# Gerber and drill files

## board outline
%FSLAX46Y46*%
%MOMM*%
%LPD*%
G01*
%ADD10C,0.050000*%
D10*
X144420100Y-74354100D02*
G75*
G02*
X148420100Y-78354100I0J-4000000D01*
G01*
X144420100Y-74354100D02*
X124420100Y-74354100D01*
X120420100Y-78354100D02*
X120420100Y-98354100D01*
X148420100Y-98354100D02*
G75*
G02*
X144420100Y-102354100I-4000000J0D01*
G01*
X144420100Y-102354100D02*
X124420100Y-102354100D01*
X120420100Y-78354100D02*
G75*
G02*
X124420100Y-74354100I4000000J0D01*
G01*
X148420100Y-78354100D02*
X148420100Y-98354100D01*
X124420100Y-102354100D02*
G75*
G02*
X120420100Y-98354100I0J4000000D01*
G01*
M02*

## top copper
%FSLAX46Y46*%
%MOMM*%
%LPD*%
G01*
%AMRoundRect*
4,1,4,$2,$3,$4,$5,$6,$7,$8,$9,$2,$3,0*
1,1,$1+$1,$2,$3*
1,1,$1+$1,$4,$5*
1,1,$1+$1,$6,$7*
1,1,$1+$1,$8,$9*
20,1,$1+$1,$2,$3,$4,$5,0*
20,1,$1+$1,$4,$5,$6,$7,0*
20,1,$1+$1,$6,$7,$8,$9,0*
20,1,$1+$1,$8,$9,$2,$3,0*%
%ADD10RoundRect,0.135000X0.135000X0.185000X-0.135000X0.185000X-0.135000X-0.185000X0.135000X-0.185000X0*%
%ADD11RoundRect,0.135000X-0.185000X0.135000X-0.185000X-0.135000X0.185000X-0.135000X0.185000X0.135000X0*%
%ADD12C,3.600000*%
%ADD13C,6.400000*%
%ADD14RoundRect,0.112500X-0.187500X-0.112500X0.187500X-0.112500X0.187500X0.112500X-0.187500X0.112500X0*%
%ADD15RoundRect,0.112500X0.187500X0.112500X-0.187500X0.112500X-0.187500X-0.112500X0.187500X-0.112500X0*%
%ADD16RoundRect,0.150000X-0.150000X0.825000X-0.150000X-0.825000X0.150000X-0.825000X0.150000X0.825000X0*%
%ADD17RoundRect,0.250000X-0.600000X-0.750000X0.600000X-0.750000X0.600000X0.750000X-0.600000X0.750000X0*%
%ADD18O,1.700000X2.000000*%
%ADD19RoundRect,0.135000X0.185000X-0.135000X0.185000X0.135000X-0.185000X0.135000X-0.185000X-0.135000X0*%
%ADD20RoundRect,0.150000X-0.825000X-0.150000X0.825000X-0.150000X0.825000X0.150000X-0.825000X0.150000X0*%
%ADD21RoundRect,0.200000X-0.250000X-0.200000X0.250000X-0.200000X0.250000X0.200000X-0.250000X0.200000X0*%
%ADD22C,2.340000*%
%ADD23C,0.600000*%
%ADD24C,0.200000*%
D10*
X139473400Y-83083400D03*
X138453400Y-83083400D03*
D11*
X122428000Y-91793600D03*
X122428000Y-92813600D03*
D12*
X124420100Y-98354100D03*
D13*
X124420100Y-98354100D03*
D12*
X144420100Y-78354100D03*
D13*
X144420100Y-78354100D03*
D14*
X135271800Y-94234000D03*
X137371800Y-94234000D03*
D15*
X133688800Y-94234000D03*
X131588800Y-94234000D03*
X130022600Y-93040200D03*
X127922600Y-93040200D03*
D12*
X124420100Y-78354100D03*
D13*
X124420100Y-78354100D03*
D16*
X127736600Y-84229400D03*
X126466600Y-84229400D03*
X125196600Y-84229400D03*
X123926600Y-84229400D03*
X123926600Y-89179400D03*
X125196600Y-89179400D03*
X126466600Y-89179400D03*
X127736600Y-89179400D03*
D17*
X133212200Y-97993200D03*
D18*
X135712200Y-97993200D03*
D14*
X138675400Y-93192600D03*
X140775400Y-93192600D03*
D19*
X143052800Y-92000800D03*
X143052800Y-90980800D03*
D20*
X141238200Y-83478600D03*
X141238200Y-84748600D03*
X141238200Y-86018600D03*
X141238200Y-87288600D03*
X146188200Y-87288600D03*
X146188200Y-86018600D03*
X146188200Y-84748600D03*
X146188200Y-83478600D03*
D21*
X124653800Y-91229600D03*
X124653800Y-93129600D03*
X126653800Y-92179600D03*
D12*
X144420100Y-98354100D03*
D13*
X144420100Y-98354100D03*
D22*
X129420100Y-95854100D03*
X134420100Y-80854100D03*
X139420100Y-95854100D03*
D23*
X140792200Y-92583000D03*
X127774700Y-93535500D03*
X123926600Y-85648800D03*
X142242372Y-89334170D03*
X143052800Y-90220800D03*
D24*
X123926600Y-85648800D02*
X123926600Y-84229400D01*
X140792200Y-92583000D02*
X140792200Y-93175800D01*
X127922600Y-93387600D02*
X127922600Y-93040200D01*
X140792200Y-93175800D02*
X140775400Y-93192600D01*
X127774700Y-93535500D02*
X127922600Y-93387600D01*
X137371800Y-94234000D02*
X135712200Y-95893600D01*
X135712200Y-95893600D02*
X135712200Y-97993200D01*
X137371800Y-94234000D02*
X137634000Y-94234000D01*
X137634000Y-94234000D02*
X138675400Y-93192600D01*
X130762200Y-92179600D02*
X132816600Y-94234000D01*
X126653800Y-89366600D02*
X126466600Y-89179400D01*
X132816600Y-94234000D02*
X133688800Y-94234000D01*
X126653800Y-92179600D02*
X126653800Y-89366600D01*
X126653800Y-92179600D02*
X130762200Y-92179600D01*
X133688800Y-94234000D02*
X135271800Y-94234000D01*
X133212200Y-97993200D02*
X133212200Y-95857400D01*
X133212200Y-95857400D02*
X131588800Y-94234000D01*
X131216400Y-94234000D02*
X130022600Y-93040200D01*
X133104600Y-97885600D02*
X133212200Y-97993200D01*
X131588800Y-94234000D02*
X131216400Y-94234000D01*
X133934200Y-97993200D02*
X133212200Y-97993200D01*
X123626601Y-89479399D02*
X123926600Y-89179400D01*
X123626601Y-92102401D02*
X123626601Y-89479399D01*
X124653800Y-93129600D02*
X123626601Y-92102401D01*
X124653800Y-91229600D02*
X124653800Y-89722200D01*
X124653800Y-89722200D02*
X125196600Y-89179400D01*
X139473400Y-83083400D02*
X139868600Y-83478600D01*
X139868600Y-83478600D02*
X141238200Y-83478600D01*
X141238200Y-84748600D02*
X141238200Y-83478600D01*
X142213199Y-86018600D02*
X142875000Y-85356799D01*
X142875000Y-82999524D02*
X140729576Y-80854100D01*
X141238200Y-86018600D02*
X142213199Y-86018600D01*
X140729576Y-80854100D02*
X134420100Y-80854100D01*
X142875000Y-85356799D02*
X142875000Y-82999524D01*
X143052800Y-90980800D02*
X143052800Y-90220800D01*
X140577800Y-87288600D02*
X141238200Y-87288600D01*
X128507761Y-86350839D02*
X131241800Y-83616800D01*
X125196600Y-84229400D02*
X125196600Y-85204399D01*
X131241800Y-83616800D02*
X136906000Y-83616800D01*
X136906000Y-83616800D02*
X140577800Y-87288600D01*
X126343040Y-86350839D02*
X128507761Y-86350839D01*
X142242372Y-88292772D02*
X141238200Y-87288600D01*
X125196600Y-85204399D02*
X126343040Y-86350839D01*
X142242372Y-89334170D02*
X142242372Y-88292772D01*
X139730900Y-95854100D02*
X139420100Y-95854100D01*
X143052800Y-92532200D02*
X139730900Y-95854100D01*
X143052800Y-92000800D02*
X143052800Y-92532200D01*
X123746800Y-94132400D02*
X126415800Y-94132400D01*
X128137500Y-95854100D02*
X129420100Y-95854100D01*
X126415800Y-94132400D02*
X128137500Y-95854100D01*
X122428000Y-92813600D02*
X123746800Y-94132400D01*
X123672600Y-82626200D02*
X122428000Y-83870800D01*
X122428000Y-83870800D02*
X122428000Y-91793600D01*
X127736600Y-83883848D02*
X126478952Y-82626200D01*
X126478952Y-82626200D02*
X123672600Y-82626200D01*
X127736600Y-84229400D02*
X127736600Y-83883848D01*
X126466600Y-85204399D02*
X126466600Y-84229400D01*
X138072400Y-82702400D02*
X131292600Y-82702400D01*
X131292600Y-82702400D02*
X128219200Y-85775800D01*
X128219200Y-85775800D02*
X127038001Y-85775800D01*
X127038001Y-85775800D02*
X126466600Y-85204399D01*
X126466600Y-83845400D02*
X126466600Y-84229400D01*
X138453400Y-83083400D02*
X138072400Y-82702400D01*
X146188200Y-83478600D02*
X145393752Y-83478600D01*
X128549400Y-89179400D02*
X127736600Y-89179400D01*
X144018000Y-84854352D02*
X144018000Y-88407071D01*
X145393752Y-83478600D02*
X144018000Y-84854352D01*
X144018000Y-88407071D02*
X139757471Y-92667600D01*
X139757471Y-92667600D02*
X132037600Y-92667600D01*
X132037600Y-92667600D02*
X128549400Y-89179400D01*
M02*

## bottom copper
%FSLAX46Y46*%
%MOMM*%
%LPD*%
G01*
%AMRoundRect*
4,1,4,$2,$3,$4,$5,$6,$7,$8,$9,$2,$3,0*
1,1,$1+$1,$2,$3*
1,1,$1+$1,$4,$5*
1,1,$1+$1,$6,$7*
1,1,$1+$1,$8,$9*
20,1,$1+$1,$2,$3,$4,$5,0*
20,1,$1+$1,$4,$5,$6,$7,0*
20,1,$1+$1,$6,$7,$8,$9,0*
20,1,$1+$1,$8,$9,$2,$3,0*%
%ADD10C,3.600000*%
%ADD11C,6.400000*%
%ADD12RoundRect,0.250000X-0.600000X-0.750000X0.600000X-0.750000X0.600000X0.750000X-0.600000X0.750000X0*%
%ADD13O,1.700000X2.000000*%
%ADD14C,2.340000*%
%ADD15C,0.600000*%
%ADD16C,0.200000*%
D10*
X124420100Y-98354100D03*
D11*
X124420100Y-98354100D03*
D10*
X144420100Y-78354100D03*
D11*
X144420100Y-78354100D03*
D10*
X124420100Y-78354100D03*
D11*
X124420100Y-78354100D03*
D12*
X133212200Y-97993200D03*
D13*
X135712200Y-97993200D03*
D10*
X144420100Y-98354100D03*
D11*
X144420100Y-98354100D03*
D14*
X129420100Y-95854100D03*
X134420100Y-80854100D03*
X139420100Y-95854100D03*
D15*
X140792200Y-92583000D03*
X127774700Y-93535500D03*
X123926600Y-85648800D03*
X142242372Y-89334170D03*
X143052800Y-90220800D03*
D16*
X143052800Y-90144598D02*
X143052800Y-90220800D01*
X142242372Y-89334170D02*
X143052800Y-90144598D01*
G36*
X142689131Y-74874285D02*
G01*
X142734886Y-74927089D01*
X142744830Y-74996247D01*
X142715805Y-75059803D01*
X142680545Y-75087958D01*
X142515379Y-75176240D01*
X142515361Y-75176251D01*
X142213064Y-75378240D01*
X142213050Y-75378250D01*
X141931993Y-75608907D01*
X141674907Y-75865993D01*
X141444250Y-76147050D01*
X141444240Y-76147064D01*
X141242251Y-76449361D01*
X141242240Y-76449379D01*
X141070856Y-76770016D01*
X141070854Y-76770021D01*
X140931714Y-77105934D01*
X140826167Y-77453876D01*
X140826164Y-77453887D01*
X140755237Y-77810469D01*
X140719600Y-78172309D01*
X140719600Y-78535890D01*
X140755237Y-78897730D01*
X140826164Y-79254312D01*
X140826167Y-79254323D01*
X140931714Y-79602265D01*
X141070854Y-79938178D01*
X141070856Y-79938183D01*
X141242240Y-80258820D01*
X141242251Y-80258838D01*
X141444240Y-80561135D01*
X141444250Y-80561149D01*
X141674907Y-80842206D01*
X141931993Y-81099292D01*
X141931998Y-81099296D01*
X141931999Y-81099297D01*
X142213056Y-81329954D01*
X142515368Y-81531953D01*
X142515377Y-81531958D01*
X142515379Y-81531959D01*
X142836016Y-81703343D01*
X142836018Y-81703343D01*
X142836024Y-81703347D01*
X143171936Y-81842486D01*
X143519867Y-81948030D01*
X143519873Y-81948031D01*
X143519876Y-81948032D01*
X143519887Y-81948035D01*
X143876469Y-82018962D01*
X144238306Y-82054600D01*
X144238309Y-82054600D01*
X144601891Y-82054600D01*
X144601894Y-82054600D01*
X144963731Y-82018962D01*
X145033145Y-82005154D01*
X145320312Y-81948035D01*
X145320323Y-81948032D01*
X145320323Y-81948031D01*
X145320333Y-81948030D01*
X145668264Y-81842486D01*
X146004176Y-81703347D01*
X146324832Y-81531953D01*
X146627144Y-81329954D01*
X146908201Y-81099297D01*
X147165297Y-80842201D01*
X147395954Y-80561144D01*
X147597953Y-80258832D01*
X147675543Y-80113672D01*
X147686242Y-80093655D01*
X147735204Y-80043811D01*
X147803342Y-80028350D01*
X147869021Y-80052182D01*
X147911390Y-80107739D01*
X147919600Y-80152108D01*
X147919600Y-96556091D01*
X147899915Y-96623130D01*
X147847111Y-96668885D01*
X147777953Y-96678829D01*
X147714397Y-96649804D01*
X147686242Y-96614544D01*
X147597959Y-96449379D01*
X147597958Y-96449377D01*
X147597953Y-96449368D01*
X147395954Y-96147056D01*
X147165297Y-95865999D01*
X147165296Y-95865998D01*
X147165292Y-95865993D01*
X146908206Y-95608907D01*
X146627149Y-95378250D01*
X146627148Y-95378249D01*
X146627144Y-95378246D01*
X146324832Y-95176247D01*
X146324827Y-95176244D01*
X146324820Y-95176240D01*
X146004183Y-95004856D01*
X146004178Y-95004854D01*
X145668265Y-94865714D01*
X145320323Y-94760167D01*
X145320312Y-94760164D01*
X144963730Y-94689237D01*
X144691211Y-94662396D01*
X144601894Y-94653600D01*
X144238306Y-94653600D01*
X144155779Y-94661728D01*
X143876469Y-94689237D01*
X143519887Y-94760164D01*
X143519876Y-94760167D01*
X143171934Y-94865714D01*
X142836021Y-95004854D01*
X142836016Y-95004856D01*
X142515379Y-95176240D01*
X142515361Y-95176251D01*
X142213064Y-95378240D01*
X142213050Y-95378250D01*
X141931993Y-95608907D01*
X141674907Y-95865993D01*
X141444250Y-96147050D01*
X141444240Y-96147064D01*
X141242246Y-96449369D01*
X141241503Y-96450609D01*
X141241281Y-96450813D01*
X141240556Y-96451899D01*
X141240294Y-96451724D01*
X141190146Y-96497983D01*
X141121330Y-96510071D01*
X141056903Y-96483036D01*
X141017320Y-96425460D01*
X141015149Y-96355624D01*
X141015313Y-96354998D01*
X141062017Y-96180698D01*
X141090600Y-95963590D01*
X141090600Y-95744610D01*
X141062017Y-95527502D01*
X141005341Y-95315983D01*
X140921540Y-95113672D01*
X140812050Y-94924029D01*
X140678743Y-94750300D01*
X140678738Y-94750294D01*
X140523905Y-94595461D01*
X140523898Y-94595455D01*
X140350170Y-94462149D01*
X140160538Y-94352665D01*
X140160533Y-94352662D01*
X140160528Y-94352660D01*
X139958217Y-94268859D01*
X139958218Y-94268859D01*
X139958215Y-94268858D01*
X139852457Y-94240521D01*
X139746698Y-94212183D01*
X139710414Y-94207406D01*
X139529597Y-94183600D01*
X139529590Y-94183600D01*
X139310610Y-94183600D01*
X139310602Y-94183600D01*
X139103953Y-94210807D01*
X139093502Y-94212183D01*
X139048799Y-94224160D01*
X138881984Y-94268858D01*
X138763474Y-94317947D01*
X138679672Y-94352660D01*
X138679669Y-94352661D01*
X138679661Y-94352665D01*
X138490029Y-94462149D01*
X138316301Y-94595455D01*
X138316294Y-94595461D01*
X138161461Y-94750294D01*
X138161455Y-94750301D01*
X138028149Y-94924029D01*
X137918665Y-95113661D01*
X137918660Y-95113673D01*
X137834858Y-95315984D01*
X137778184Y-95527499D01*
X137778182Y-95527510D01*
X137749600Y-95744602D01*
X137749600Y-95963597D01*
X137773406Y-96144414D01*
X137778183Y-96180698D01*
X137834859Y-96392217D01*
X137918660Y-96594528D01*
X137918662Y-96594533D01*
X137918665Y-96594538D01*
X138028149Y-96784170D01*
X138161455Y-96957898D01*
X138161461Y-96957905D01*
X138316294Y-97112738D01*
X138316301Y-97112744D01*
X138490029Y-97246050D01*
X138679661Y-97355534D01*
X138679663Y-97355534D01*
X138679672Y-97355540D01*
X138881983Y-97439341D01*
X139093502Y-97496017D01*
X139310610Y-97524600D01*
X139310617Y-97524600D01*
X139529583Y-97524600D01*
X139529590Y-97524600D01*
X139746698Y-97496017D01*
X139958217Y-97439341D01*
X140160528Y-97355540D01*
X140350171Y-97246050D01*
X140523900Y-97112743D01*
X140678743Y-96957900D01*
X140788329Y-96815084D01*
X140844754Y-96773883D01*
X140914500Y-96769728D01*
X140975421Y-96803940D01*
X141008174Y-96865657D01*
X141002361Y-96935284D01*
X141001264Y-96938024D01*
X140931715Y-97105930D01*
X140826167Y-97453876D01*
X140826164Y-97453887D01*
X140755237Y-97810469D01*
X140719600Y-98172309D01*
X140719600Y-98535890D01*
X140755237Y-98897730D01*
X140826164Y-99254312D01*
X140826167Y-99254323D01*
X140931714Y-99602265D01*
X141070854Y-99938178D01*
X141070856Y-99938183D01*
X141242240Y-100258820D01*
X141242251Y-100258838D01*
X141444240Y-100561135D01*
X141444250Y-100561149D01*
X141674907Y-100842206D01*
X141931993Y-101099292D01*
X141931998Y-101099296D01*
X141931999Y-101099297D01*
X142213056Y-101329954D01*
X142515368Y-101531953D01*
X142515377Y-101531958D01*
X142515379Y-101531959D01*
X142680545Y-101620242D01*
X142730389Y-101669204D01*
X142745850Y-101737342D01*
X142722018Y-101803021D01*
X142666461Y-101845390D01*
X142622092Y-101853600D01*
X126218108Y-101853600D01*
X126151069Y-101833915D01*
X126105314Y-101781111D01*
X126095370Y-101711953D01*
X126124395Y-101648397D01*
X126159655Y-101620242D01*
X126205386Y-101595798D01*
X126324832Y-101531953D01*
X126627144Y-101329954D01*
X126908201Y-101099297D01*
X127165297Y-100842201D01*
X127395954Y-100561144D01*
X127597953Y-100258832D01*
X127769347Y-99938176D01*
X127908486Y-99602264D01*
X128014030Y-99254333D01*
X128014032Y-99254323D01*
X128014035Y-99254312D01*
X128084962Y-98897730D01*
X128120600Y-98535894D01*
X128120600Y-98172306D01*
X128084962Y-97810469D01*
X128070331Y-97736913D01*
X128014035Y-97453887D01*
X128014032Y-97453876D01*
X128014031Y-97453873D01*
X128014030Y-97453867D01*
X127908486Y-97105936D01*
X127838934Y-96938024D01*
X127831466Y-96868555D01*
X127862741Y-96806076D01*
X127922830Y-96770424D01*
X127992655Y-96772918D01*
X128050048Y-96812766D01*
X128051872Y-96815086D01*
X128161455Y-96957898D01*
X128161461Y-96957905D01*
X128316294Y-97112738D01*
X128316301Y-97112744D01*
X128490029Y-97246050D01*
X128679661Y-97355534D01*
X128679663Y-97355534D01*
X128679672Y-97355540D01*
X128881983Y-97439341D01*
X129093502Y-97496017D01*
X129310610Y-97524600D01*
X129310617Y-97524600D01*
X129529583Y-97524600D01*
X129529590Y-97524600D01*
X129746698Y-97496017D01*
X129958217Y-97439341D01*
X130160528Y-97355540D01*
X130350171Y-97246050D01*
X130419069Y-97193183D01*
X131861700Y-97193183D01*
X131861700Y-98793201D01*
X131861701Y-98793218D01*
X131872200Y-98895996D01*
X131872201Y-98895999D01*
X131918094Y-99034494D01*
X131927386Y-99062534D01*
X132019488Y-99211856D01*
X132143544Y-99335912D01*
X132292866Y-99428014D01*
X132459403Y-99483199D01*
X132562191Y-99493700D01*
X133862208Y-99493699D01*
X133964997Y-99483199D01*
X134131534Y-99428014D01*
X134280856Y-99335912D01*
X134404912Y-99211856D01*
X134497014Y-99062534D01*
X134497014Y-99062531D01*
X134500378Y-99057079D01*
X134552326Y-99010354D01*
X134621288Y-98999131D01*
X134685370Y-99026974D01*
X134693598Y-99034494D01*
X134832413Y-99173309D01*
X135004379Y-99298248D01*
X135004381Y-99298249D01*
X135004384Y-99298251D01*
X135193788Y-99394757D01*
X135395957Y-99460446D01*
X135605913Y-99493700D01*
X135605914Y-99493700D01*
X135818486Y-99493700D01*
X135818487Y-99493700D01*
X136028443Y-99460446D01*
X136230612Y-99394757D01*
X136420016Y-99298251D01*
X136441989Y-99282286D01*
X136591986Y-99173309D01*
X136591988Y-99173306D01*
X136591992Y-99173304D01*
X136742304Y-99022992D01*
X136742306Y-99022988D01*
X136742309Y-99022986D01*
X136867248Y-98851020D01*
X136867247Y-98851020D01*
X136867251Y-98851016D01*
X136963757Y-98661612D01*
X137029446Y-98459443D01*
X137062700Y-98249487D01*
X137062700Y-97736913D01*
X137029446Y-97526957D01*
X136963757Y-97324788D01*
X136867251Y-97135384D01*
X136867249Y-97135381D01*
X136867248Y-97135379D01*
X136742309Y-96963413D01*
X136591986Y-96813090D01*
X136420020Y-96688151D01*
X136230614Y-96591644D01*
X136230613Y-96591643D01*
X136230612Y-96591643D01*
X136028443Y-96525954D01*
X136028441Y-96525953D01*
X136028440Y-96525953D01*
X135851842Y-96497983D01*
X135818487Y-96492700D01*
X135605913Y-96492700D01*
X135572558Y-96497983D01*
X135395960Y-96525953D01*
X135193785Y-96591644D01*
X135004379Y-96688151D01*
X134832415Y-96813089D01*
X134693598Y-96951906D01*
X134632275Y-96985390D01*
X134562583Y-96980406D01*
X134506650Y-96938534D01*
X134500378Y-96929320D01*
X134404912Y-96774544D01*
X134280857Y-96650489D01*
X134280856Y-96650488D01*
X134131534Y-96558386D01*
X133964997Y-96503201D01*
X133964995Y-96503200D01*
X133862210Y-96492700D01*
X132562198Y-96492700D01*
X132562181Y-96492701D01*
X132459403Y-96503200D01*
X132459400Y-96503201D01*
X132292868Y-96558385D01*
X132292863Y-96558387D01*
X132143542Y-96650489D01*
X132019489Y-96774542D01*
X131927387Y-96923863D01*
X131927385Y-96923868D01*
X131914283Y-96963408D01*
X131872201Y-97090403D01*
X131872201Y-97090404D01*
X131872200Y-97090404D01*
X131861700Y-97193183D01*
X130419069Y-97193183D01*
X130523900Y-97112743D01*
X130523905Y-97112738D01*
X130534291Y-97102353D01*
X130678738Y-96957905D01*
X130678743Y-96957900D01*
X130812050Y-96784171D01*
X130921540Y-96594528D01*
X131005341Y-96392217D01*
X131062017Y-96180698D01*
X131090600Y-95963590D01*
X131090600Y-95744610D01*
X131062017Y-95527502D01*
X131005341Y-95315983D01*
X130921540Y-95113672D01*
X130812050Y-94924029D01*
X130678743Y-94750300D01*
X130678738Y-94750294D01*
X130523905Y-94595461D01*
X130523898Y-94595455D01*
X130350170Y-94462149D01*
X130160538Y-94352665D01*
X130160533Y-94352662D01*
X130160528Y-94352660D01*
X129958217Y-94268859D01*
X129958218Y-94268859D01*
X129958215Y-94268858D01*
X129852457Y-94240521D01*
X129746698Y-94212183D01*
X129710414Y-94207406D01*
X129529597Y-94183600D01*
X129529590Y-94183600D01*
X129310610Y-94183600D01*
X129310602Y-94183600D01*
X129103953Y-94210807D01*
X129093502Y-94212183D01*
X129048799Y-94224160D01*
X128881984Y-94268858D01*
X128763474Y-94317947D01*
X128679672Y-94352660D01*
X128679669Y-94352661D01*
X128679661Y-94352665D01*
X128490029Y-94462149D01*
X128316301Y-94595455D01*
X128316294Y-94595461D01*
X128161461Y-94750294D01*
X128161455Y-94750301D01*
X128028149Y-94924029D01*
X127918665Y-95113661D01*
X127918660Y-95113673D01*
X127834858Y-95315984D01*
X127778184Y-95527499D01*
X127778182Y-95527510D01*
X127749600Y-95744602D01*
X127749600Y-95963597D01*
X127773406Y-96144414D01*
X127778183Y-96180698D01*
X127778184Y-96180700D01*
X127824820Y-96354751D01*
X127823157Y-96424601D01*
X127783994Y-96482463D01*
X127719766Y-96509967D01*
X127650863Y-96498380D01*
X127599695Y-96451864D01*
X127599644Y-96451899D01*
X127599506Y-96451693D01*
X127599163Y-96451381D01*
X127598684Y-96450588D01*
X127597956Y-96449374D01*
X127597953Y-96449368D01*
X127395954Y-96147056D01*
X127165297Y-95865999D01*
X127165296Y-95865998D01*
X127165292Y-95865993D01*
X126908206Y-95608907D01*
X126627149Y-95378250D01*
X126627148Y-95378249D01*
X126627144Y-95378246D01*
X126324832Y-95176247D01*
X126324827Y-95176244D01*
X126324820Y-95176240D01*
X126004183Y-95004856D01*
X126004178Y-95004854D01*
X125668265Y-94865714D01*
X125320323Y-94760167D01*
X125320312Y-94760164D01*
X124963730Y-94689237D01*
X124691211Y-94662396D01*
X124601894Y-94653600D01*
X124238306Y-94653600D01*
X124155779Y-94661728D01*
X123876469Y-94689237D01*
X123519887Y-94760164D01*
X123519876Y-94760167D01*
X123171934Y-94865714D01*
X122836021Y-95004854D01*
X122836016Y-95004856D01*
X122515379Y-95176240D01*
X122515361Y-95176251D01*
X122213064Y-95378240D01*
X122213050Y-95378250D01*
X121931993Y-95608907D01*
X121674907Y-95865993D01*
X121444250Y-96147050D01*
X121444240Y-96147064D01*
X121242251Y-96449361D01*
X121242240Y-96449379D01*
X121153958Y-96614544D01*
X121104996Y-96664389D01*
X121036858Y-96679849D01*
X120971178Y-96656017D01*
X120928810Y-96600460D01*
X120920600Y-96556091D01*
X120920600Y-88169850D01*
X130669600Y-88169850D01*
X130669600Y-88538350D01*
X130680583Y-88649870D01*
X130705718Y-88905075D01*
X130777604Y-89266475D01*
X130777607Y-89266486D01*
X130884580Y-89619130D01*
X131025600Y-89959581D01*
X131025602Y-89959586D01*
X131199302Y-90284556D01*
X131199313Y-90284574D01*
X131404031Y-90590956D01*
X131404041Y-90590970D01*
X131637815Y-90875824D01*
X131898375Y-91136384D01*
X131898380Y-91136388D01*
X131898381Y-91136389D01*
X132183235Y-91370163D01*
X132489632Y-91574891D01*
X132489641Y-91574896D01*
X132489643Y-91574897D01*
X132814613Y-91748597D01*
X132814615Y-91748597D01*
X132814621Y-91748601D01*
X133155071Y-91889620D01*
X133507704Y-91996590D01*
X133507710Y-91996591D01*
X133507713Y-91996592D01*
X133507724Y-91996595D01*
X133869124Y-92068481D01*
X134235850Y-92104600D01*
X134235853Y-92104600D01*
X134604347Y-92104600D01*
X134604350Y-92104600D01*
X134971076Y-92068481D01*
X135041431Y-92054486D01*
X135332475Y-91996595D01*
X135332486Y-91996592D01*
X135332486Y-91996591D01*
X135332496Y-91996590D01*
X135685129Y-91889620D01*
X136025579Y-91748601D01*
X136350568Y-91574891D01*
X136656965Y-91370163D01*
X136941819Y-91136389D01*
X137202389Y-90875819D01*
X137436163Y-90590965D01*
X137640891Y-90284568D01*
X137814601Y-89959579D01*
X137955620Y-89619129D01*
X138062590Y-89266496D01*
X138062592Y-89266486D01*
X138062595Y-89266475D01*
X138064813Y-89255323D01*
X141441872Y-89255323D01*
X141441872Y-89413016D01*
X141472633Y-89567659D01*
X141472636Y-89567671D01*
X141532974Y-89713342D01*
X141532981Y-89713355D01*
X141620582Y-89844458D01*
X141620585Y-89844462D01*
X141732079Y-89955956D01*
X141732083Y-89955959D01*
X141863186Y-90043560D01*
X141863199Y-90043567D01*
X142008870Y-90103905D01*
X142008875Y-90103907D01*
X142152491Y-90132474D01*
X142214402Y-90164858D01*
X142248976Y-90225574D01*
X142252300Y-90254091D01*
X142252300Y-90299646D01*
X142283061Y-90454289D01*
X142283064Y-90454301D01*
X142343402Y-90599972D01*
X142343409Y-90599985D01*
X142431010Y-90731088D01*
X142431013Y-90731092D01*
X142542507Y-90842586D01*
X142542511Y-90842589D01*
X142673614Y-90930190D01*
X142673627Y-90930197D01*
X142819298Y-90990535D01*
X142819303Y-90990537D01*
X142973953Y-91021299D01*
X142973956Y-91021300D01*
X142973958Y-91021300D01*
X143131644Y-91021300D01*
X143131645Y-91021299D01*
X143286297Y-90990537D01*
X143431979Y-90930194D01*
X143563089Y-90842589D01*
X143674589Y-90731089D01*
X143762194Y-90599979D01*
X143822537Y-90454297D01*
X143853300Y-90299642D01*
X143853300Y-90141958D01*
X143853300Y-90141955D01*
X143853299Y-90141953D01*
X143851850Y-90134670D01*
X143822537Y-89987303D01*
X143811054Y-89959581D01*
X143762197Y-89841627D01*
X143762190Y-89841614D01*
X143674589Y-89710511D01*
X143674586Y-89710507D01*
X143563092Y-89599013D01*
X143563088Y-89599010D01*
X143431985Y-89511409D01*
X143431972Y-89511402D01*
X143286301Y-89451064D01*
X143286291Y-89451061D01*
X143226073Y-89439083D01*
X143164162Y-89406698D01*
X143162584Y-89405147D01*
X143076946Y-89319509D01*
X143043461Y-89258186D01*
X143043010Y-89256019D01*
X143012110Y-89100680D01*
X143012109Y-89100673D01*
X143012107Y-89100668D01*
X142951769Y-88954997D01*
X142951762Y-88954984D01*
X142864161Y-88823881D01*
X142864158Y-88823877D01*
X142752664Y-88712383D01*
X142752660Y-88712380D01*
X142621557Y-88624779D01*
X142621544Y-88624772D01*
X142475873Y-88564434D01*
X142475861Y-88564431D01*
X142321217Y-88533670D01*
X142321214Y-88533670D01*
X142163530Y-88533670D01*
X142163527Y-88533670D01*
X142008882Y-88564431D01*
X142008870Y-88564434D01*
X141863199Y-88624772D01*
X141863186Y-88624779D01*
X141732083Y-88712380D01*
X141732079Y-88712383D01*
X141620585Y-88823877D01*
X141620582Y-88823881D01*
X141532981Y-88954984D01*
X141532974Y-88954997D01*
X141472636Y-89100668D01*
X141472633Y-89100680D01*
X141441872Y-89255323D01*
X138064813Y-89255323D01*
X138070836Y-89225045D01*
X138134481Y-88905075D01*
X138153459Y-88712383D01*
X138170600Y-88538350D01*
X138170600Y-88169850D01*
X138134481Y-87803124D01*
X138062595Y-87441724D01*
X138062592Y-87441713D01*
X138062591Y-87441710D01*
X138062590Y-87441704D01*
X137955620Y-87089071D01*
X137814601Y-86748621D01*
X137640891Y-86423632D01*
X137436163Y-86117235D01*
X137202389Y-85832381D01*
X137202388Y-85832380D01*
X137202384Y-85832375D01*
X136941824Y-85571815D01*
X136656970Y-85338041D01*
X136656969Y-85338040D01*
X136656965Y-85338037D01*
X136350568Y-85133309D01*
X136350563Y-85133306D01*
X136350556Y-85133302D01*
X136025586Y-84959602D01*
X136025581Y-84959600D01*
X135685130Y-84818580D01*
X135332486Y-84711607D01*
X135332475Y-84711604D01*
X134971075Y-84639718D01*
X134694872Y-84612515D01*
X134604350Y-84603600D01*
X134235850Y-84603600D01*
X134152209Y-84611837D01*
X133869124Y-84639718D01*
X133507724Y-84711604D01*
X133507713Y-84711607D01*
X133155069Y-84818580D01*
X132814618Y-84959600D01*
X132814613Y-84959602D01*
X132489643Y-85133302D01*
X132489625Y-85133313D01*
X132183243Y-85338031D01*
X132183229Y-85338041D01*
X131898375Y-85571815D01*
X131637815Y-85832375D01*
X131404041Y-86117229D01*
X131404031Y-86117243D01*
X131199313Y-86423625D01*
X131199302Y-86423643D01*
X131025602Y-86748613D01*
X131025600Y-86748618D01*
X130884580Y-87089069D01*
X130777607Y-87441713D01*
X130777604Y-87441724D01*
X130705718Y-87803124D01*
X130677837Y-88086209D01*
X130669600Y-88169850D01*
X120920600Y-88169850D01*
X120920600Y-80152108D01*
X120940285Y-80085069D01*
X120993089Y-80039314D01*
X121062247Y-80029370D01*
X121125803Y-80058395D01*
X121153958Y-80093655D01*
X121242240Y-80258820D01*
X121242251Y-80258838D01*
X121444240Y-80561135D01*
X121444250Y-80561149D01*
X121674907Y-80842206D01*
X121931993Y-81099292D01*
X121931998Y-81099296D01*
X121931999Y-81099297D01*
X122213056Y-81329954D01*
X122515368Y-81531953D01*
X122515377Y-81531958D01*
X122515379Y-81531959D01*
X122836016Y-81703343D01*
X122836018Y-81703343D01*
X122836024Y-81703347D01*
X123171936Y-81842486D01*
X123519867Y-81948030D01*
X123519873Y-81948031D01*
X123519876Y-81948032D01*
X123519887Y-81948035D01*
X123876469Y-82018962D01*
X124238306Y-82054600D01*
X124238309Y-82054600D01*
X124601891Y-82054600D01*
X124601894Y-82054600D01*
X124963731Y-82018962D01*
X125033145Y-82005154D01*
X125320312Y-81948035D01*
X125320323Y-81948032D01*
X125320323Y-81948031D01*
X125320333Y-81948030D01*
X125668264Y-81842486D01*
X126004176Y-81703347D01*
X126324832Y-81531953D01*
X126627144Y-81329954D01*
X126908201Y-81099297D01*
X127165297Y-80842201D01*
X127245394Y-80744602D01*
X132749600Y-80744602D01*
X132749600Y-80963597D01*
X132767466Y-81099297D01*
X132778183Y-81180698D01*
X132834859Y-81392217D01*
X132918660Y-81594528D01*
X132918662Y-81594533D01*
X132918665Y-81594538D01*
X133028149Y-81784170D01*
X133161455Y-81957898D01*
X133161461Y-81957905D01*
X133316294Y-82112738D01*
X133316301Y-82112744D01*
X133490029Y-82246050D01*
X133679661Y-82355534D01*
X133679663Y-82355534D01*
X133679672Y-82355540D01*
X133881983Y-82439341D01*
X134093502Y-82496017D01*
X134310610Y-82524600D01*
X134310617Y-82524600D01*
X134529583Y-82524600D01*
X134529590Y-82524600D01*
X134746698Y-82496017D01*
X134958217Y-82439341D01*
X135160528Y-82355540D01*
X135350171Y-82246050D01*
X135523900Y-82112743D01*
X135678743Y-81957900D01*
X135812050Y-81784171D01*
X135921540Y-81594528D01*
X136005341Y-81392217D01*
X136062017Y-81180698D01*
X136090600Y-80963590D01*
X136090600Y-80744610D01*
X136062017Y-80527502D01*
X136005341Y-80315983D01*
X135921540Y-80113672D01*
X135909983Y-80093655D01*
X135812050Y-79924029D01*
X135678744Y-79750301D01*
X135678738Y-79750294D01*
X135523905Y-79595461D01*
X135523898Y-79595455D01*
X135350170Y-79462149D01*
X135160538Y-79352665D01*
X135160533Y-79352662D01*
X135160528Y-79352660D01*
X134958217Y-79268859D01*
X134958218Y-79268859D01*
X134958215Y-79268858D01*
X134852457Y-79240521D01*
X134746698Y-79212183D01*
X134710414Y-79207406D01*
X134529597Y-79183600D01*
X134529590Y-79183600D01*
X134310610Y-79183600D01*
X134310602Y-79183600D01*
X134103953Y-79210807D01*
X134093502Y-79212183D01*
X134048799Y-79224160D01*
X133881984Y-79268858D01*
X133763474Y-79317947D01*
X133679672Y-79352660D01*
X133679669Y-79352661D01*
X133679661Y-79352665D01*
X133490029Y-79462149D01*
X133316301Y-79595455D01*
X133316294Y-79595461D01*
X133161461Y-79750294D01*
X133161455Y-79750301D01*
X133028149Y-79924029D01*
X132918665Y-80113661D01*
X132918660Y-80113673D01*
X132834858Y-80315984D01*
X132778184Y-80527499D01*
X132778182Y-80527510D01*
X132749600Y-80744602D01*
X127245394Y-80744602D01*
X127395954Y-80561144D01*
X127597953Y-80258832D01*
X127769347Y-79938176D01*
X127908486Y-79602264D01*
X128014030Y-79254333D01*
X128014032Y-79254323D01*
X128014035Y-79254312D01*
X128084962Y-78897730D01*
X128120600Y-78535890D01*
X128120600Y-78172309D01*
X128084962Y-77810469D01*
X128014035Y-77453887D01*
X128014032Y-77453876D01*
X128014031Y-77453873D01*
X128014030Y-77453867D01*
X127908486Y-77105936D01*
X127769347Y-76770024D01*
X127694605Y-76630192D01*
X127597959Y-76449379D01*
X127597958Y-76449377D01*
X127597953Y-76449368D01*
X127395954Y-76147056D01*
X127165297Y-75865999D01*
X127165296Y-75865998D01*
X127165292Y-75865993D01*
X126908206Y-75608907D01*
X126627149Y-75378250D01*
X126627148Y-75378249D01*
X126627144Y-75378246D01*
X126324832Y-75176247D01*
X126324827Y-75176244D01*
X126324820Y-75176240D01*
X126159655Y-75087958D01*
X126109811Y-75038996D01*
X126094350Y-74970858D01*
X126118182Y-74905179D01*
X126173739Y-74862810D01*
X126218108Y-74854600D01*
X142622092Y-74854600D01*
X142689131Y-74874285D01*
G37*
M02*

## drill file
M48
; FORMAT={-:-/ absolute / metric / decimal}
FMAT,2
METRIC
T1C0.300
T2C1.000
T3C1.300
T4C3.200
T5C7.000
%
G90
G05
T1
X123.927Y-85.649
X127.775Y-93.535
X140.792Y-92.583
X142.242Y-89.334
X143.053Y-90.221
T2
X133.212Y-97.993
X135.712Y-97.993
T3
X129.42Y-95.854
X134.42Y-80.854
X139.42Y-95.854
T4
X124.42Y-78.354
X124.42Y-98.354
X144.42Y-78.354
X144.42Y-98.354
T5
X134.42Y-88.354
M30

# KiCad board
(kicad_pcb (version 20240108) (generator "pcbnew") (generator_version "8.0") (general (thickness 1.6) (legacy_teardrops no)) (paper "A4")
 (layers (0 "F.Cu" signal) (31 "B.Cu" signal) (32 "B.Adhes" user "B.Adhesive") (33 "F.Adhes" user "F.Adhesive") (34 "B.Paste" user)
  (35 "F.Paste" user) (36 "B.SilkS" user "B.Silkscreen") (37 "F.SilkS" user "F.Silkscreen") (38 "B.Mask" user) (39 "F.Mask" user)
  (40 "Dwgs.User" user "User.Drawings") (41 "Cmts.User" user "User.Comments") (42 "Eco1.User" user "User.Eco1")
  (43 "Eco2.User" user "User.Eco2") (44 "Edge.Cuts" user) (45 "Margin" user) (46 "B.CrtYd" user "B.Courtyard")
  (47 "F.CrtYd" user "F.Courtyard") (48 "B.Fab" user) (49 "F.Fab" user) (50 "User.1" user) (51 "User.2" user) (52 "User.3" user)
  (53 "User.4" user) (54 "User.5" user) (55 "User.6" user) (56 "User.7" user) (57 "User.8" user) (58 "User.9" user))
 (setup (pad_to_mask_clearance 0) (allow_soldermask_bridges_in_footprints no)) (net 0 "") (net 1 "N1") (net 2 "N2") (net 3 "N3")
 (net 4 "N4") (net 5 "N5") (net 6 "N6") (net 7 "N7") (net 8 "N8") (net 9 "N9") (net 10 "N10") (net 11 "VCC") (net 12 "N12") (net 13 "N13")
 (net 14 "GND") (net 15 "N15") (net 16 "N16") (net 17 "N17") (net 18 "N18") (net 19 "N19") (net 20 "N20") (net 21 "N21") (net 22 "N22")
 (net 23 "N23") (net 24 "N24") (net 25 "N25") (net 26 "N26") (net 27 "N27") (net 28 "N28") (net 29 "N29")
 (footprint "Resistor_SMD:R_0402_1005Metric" (layer "F.Cu") (at 138.9634 83.0834 180)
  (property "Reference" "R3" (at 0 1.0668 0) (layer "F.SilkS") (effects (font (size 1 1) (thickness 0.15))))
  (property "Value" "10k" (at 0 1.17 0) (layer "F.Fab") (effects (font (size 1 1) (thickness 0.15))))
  (pad "1" smd roundrect (at -0.51 0 180) (size 0.54 0.64) (layers "F.Cu" "F.Paste" "F.Mask") (roundrect_rratio 0.25) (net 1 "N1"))
  (pad "2" smd roundrect (at 0.51 0 180) (size 0.54 0.64) (layers "F.Cu" "F.Paste" "F.Mask") (roundrect_rratio 0.25) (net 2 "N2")))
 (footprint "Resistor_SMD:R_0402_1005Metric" (layer "F.Cu") (at 122.428 92.3036 -90)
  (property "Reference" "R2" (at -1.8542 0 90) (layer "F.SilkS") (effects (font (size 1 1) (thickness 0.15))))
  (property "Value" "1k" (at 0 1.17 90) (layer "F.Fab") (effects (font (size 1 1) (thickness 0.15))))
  (pad "1" smd roundrect (at -0.51 0 270) (size 0.54 0.64) (layers "F.Cu" "F.Paste" "F.Mask") (roundrect_rratio 0.25) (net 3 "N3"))
  (pad "2" smd roundrect (at 0.51 0 270) (size 0.54 0.64) (layers "F.Cu" "F.Paste" "F.Mask") (roundrect_rratio 0.25) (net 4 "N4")))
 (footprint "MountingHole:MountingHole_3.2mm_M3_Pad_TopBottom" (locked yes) (layer "F.Cu") (at 124.4201 98.3541)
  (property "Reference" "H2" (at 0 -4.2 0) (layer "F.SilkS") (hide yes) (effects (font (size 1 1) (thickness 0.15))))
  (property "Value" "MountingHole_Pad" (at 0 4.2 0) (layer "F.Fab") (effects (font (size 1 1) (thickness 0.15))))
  (pad "1" thru_hole circle (at 0 0) (size 3.6 3.6) (drill 3.2) (layers "*.Cu" "*.Mask") (remove_unused_layers no) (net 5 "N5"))
  (pad "1" connect circle (at 0 0) (size 6.4 6.4) (layers "F.Cu" "F.Mask") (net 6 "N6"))
  (pad "1" connect circle (at 0 0) (size 6.4 6.4) (layers "B.Cu" "B.Mask") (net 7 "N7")))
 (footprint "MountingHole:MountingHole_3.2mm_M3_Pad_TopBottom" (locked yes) (layer "F.Cu") (at 144.4201 78.3541)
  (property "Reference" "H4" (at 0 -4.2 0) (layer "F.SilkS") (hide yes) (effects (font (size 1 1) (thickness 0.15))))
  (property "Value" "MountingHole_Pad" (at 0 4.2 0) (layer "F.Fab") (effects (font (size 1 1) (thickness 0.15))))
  (pad "1" thru_hole circle (at 0 0) (size 3.6 3.6) (drill 3.2) (layers "*.Cu" "*.Mask") (remove_unused_layers no) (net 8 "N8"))
  (pad "1" connect circle (at 0 0) (size 6.4 6.4) (layers "F.Cu" "F.Mask") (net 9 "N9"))
  (pad "1" connect circle (at 0 0) (size 6.4 6.4) (layers "B.Cu" "B.Mask") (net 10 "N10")))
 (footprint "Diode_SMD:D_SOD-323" (layer "F.Cu") (at 136.3218 94.234)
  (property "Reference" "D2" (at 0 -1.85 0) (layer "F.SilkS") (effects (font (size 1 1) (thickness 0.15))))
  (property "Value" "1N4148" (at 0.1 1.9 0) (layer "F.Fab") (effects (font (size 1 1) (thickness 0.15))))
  (pad "1" smd roundrect (at -1.05 0) (size 0.6 0.45) (layers "F.Cu" "F.Paste" "F.Mask") (roundrect_rratio 0.25) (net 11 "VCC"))
  (pad "2" smd roundrect (at 1.05 0) (size 0.6 0.45) (layers "F.Cu" "F.Paste" "F.Mask") (roundrect_rratio 0.25) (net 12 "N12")))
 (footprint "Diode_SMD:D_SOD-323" (layer "F.Cu") (at 132.6388 94.234 180)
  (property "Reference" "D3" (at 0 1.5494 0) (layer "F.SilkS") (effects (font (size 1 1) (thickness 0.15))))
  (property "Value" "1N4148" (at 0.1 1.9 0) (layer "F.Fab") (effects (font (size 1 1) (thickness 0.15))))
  (pad "1" smd roundrect (at -1.05 0 180) (size 0.6 0.45) (layers "F.Cu" "F.Paste" "F.Mask") (roundrect_rratio 0.25) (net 11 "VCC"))
  (pad "2" smd roundrect (at 1.05 0 180) (size 0.6 0.45) (layers "F.Cu" "F.Paste" "F.Mask") (roundrect_rratio 0.25) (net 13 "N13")))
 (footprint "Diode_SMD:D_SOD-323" (layer "F.Cu") (at 128.9726 93.0402 180)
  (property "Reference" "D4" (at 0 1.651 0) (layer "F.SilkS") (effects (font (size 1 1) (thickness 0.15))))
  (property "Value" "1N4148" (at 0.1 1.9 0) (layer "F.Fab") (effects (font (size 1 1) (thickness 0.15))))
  (pad "1" smd roundrect (at -1.05 0 180) (size 0.6 0.45) (layers "F.Cu" "F.Paste" "F.Mask") (roundrect_rratio 0.25) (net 13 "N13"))
  (pad "2" smd roundrect (at 1.05 0 180) (size 0.6 0.45) (layers "F.Cu" "F.Paste" "F.Mask") (roundrect_rratio 0.25) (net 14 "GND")))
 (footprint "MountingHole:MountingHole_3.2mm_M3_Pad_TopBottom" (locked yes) (layer "F.Cu") (at 124.4201 78.3541)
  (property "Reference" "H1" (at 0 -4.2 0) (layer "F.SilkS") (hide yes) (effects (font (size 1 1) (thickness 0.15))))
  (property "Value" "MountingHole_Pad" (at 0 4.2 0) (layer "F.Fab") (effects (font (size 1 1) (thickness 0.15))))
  (pad "1" thru_hole circle (at 0 0) (size 3.6 3.6) (drill 3.2) (layers "*.Cu" "*.Mask") (remove_unused_layers no) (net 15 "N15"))
  (pad "1" connect circle (at 0 0) (size 6.4 6.4) (layers "F.Cu" "F.Mask") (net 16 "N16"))
  (pad "1" connect circle (at 0 0) (size 6.4 6.4) (layers "B.Cu" "B.Mask") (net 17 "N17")))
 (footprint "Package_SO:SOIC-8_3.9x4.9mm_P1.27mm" (layer "F.Cu") (at 125.8316 86.7044 -90)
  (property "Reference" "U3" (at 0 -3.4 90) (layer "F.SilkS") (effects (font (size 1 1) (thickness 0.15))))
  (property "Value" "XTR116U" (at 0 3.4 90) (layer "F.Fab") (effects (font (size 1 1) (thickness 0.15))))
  (pad "1" smd roundrect (at -2.475 -1.905 270) (size 1.95 0.6) (layers "F.Cu" "F.Paste" "F.Mask") (roundrect_rratio 0.25) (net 3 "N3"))
  (pad "2" smd roundrect (at -2.475 -0.635 270) (size 1.95 0.6) (layers "F.Cu" "F.Paste" "F.Mask") (roundrect_rratio 0.25) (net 2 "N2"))
  (pad "3" smd roundrect (at -2.475 0.635 270) (size 1.95 0.6) (layers "F.Cu" "F.Paste" "F.Mask") (roundrect_rratio 0.25) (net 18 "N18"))
  (pad "4" smd roundrect (at -2.475 1.905 270) (size 1.95 0.6) (layers "F.Cu" "F.Paste" "F.Mask") (roundrect_rratio 0.25) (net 14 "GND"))
  (pad "5" smd roundrect (at 2.475 1.905 270) (size 1.95 0.6) (layers "F.Cu" "F.Paste" "F.Mask") (roundrect_rratio 0.25) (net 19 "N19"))
  (pad "6" smd roundrect (at 2.475 0.635 270) (size 1.95 0.6) (layers "F.Cu" "F.Paste" "F.Mask") (roundrect_rratio 0.25) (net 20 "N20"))
  (pad "7" smd roundrect (at 2.475 -0.635 270) (size 1.95 0.6) (layers "F.Cu" "F.Paste" "F.Mask") (roundrect_rratio 0.25) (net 11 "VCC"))
  (pad "8" smd roundrect (at 2.475 -1.905 270) (size 1.95 0.6) (layers "F.Cu" "F.Paste" "F.Mask") (roundrect_rratio 0.25) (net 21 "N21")))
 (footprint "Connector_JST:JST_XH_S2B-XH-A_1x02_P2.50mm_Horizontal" (layer "F.Cu") (at 133.2122 97.9932)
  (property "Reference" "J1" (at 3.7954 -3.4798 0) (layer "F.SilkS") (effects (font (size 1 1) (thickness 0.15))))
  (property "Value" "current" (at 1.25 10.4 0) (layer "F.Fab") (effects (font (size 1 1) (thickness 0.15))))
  (pad "1" thru_hole roundrect (at 0 0) (size 1.7 2) (drill 1) (layers "*.Cu" "*.Mask") (remove_unused_layers no)
   (roundrect_rratio 0.147059) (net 13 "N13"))
  (pad "2" thru_hole oval (at 2.5 0) (size 1.7 2) (drill 1) (layers "*.Cu" "*.Mask") (remove_unused_layers no) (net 12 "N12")))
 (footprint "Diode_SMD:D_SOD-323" (layer "F.Cu") (at 139.7254 93.1926)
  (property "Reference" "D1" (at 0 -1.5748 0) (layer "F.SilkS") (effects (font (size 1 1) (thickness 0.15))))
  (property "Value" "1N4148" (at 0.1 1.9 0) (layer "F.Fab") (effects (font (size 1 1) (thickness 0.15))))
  (pad "1" smd roundrect (at -1.05 0) (size 0.6 0.45) (layers "F.Cu" "F.Paste" "F.Mask") (roundrect_rratio 0.25) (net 12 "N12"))
  (pad "2" smd roundrect (at 1.05 0) (size 0.6 0.45) (layers "F.Cu" "F.Paste" "F.Mask") (roundrect_rratio 0.25) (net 14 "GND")))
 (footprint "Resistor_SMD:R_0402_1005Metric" (layer "F.Cu") (at 143.0528 91.4908 90)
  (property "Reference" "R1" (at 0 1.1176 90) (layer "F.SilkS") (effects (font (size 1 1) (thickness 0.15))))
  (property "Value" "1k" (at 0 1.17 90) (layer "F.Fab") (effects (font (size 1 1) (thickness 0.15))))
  (pad "1" smd roundrect (at -0.51 0 90) (size 0.54 0.64) (layers "F.Cu" "F.Paste" "F.Mask") (roundrect_rratio 0.25) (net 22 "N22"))
  (pad "2" smd roundrect (at 0.51 0 90) (size 0.54 0.64) (layers "F.Cu" "F.Paste" "F.Mask") (roundrect_rratio 0.25) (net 18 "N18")))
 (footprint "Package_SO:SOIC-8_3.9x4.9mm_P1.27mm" (layer "F.Cu") (at 143.7132 85.3836)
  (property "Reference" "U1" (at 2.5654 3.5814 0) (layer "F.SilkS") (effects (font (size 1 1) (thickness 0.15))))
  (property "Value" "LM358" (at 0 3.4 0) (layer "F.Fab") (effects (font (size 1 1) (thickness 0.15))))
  (pad "1" smd roundrect (at -2.475 -1.905) (size 1.95 0.6) (layers "F.Cu" "F.Paste" "F.Mask") (roundrect_rratio 0.25) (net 1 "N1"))
  (pad "2" smd roundrect (at -2.475 -0.635) (size 1.95 0.6) (layers "F.Cu" "F.Paste" "F.Mask") (roundrect_rratio 0.25) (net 1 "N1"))
  (pad "3" smd roundrect (at -2.475 0.635) (size 1.95 0.6) (layers "F.Cu" "F.Paste" "F.Mask") (roundrect_rratio 0.25) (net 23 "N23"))
  (pad "4" smd roundrect (at -2.475 1.905) (size 1.95 0.6) (layers "F.Cu" "F.Paste" "F.Mask") (roundrect_rratio 0.25) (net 18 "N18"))
  (pad "5" smd roundrect (at 2.475 1.905) (size 1.95 0.6) (layers "F.Cu" "F.Paste" "F.Mask") (roundrect_rratio 0.25) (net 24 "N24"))
  (pad "6" smd roundrect (at 2.475 0.635) (size 1.95 0.6) (layers "F.Cu" "F.Paste" "F.Mask") (roundrect_rratio 0.25) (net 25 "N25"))
  (pad "7" smd roundrect (at 2.475 -0.635) (size 1.95 0.6) (layers "F.Cu" "F.Paste" "F.Mask") (roundrect_rratio 0.25) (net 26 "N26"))
  (pad "8" smd roundrect (at 2.475 -1.905) (size 1.95 0.6) (layers "F.Cu" "F.Paste" "F.Mask") (roundrect_rratio 0.25) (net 21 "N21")))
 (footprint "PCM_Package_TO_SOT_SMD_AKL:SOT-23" (layer "F.Cu") (at 125.6538 92.1796)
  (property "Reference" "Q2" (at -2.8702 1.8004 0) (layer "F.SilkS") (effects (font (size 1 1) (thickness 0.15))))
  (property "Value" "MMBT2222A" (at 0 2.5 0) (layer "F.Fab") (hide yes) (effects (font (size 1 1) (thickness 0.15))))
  (pad "1" smd roundrect (at -1 -0.95) (size 0.9 0.8) (layers "F.Cu" "F.Paste" "F.Mask") (roundrect_rratio 0.25) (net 20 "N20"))
  (pad "2" smd roundrect (at -1 0.95) (size 0.9 0.8) (layers "F.Cu" "F.Paste" "F.Mask") (roundrect_rratio 0.25) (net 19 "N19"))
  (pad "3" smd roundrect (at 1 0) (size 0.9 0.8) (layers "F.Cu" "F.Paste" "F.Mask") (roundrect_rratio 0.25) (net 11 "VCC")))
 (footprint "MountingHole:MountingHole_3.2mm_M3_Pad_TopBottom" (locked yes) (layer "F.Cu") (at 144.4201 98.3541)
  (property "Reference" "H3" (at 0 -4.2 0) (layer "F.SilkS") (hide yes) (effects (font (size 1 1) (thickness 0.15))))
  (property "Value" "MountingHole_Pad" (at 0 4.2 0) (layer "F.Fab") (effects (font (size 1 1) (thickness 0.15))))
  (pad "1" thru_hole circle (at 0 0) (size 3.6 3.6) (drill 3.2) (layers "*.Cu" "*.Mask") (remove_unused_layers no) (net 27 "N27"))
  (pad "1" connect circle (at 0 0) (size 6.4 6.4) (layers "F.Cu" "F.Mask") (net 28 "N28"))
  (pad "1" connect circle (at 0 0) (size 6.4 6.4) (layers "B.Cu" "B.Mask") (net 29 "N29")))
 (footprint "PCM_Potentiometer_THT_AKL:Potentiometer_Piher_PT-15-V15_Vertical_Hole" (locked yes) (layer "B.Cu") (at 129.4201 95.8541 90)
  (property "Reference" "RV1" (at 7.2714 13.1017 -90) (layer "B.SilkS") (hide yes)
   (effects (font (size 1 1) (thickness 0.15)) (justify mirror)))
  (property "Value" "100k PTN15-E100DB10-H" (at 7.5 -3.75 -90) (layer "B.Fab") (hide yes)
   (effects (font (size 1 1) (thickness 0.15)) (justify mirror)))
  (pad "" np_thru_hole circle (at 7.5 5 90) (size 7 7) (drill 7) (layers "*.Cu" "*.Mask"))
  (pad "1" thru_hole circle (at 0 0 90) (size 2.34 2.34) (drill 1.3) (layers "*.Cu" "*.Mask") (remove_unused_layers no) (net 4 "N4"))
  (pad "2" thru_hole circle (at 15 5 90) (size 2.34 2.34) (drill 1.3) (layers "*.Cu" "*.Mask") (remove_unused_layers no) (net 23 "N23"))
  (pad "3" thru_hole circle (at 0 10 90) (size 2.34 2.34) (drill 1.3) (layers "*.Cu" "*.Mask") (remove_unused_layers no) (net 22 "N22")))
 (gr_arc (start 144.4201 74.3541) (mid 147.248527 75.525673) (end 148.4201 78.3541) (stroke (width 0.05) (type default)) (layer "Edge.Cuts"))
 (gr_line (start 144.4201 74.3541) (end 124.4201 74.3541) (stroke (width 0.05) (type default)) (layer "Edge.Cuts"))
 (gr_line (start 120.4201 78.3541) (end 120.4201 98.3541) (stroke (width 0.05) (type default)) (layer "Edge.Cuts"))
 (gr_arc (start 148.4201 98.3541) (mid 147.248527 101.182527) (end 144.4201 102.3541) (stroke (width 0.05) (type default))
  (layer "Edge.Cuts"))
 (gr_line (start 144.4201 102.3541) (end 124.4201 102.3541) (stroke (width 0.05) (type default)) (layer "Edge.Cuts"))
 (gr_arc (start 120.4201 78.3541) (mid 121.591673 75.525673) (end 124.4201 74.3541) (stroke (width 0.05) (type default)) (layer "Edge.Cuts"))
 (gr_line (start 148.4201 78.3541) (end 148.4201 98.3541) (stroke (width 0.05) (type default)) (layer "Edge.Cuts"))
 (gr_arc (start 124.4201 102.3541) (mid 121.591673 101.182527) (end 120.4201 98.3541) (stroke (width 0.05) (type default))
  (layer "Edge.Cuts"))
 (segment (start 123.9266 85.6488) (end 123.9266 84.2294) (width 0.2) (layer "F.Cu") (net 14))
 (segment (start 140.7922 92.583) (end 140.7922 93.1758) (width 0.2) (layer "F.Cu") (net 14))
 (segment (start 127.9226 93.3876) (end 127.9226 93.0402) (width 0.2) (layer "F.Cu") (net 14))
 (segment (start 140.7922 93.1758) (end 140.7754 93.1926) (width 0.2) (layer "F.Cu") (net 14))
 (segment (start 127.7747 93.5355) (end 127.9226 93.3876) (width 0.2) (layer "F.Cu") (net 14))
 (via (at 140.7922 92.583) (size 0.6) (drill 0.3) (layers "F.Cu" "B.Cu") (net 14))
 (via (at 127.7747 93.5355) (size 0.6) (drill 0.3) (layers "F.Cu" "B.Cu") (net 14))
 (via (at 123.9266 85.6488) (size 0.6) (drill 0.3) (layers "F.Cu" "B.Cu") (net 14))
 (segment (start 137.3718 94.234) (end 135.7122 95.8936) (width 0.2) (layer "F.Cu") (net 12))
 (segment (start 135.7122 95.8936) (end 135.7122 97.9932) (width 0.2) (layer "F.Cu") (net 12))
 (segment (start 137.3718 94.234) (end 137.634 94.234) (width 0.2) (layer "F.Cu") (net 12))
 (segment (start 137.634 94.234) (end 138.6754 93.1926) (width 0.2) (layer "F.Cu") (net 12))
 (segment (start 130.7622 92.1796) (end 132.8166 94.234) (width 0.2) (layer "F.Cu") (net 11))
 (segment (start 126.6538 89.3666) (end 126.4666 89.1794) (width 0.2) (layer "F.Cu") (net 11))
 (segment (start 132.8166 94.234) (end 133.6888 94.234) (width 0.2) (layer "F.Cu") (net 11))
 (segment (start 126.6538 92.1796) (end 126.6538 89.3666) (width 0.2) (layer "F.Cu") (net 11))
 (segment (start 126.6538 92.1796) (end 130.7622 92.1796) (width 0.2) (layer "F.Cu") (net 11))
 (segment (start 133.6888 94.234) (end 135.2718 94.234) (width 0.2) (layer "F.Cu") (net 11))
 (segment (start 133.2122 97.9932) (end 133.2122 95.8574) (width 0.2) (layer "F.Cu") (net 13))
 (segment (start 133.2122 95.8574) (end 131.5888 94.234) (width 0.2) (layer "F.Cu") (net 13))
 (segment (start 131.2164 94.234) (end 130.0226 93.0402) (width 0.2) (layer "F.Cu") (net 13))
 (segment (start 133.1046 97.8856) (end 133.2122 97.9932) (width 0.2) (layer "F.Cu") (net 13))
 (segment (start 131.5888 94.234) (end 131.2164 94.234) (width 0.2) (layer "F.Cu") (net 13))
 (segment (start 133.9342 97.9932) (end 133.2122 97.9932) (width 0.2) (layer "F.Cu") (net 13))
 (segment (start 123.626601 89.479399) (end 123.9266 89.1794) (width 0.2) (layer "F.Cu") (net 19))
 (segment (start 123.626601 92.102401) (end 123.626601 89.479399) (width 0.2) (layer "F.Cu") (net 19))
 (segment (start 124.6538 93.1296) (end 123.626601 92.102401) (width 0.2) (layer "F.Cu") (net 19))
 (segment (start 124.6538 91.2296) (end 124.6538 89.7222) (width 0.2) (layer "F.Cu") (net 20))
 (segment (start 124.6538 89.7222) (end 125.1966 89.1794) (width 0.2) (layer "F.Cu") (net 20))
 (segment (start 139.4734 83.0834) (end 139.8686 83.4786) (width 0.2) (layer "F.Cu") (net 1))
 (segment (start 139.8686 83.4786) (end 141.2382 83.4786) (width 0.2) (layer "F.Cu") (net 1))
 (segment (start 141.2382 84.7486) (end 141.2382 83.4786) (width 0.2) (layer "F.Cu") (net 1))
 (segment (start 142.213199 86.0186) (end 142.875 85.356799) (width 0.2) (layer "F.Cu") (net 23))
 (segment (start 142.875 82.999524) (end 140.729576 80.8541) (width 0.2) (layer "F.Cu") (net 23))
 (segment (start 141.2382 86.0186) (end 142.213199 86.0186) (width 0.2) (layer "F.Cu") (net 23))
 (segment (start 140.729576 80.8541) (end 134.4201 80.8541) (width 0.2) (layer "F.Cu") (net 23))
 (segment (start 142.875 85.356799) (end 142.875 82.999524) (width 0.2) (layer "F.Cu") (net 23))
 (segment (start 143.0528 90.9808) (end 143.0528 90.2208) (width 0.2) (layer "F.Cu") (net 18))
 (segment (start 140.5778 87.2886) (end 141.2382 87.2886) (width 0.2) (layer "F.Cu") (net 18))
 (segment (start 128.507761 86.350839) (end 131.2418 83.6168) (width 0.2) (layer "F.Cu") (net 18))
 (segment (start 125.1966 84.2294) (end 125.1966 85.204399) (width 0.2) (layer "F.Cu") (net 18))
 (segment (start 131.2418 83.6168) (end 136.906 83.6168) (width 0.2) (layer "F.Cu") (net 18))
 (segment (start 136.906 83.6168) (end 140.5778 87.2886) (width 0.2) (layer "F.Cu") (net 18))
 (segment (start 126.34304 86.350839) (end 128.507761 86.350839) (width 0.2) (layer "F.Cu") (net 18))
 (segment (start 142.242372 88.292772) (end 141.2382 87.2886) (width 0.2) (layer "F.Cu") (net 18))
 (segment (start 125.1966 85.204399) (end 126.34304 86.350839) (width 0.2) (layer "F.Cu") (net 18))
 (segment (start 142.242372 89.33417) (end 142.242372 88.292772) (width 0.2) (layer "F.Cu") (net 18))
 (via (at 142.242372 89.33417) (size 0.6) (drill 0.3) (layers "F.Cu" "B.Cu") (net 18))
 (via (at 143.0528 90.2208) (size 0.6) (drill 0.3) (layers "F.Cu" "B.Cu") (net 18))
 (segment (start 143.0528 90.144598) (end 143.0528 90.2208) (width 0.2) (layer "B.Cu") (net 18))
 (segment (start 142.242372 89.33417) (end 143.0528 90.144598) (width 0.2) (layer "B.Cu") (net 18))
 (segment (start 139.7309 95.8541) (end 139.4201 95.8541) (width 0.2) (layer "F.Cu") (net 22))
 (segment (start 143.0528 92.5322) (end 139.7309 95.8541) (width 0.2) (layer "F.Cu") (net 22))
 (segment (start 143.0528 92.0008) (end 143.0528 92.5322) (width 0.2) (layer "F.Cu") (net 22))
 (segment (start 123.7468 94.1324) (end 126.4158 94.1324) (width 0.2) (layer "F.Cu") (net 4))
 (segment (start 128.1375 95.8541) (end 129.4201 95.8541) (width 0.2) (layer "F.Cu") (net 4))
 (segment (start 126.4158 94.1324) (end 128.1375 95.8541) (width 0.2) (layer "F.Cu") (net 4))
 (segment (start 122.428 92.8136) (end 123.7468 94.1324) (width 0.2) (layer "F.Cu") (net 4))
 (segment (start 123.6726 82.6262) (end 122.428 83.8708) (width 0.2) (layer "F.Cu") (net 3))
 (segment (start 122.428 83.8708) (end 122.428 91.7936) (width 0.2) (layer "F.Cu") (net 3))
 (segment (start 127.7366 83.883848) (end 126.478952 82.6262) (width 0.2) (layer "F.Cu") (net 3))
 (segment (start 126.478952 82.6262) (end 123.6726 82.6262) (width 0.2) (layer "F.Cu") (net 3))
 (segment (start 127.7366 84.2294) (end 127.7366 83.883848) (width 0.2) (layer "F.Cu") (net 3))
 (segment (start 126.4666 85.204399) (end 126.4666 84.2294) (width 0.2) (layer "F.Cu") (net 2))
 (segment (start 138.0724 82.7024) (end 131.2926 82.7024) (width 0.2) (layer "F.Cu") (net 2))
 (segment (start 131.2926 82.7024) (end 128.2192 85.7758) (width 0.2) (layer "F.Cu") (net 2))
 (segment (start 128.2192 85.7758) (end 127.038001 85.7758) (width 0.2) (layer "F.Cu") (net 2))
 (segment (start 127.038001 85.7758) (end 126.4666 85.204399) (width 0.2) (layer "F.Cu") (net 2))
 (segment (start 126.4666 83.8454) (end 126.4666 84.2294) (width 0.2) (layer "F.Cu") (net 2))
 (segment (start 138.4534 83.0834) (end 138.0724 82.7024) (width 0.2) (layer "F.Cu") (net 2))
 (segment (start 146.1882 83.4786) (end 145.393752 83.4786) (width 0.2) (layer "F.Cu") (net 21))
 (segment (start 128.5494 89.1794) (end 127.7366 89.1794) (width 0.2) (layer "F.Cu") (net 21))
 (segment (start 144.018 84.854352) (end 144.018 88.407071) (width 0.2) (layer "F.Cu") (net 21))
 (segment (start 145.393752 83.4786) (end 144.018 84.854352) (width 0.2) (layer "F.Cu") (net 21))
 (segment (start 144.018 88.407071) (end 139.757471 92.6676) (width 0.2) (layer "F.Cu") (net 21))
 (segment (start 139.757471 92.6676) (end 132.0376 92.6676) (width 0.2) (layer "F.Cu") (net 21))
 (segment (start 132.0376 92.6676) (end 128.5494 89.1794) (width 0.2) (layer "F.Cu") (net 21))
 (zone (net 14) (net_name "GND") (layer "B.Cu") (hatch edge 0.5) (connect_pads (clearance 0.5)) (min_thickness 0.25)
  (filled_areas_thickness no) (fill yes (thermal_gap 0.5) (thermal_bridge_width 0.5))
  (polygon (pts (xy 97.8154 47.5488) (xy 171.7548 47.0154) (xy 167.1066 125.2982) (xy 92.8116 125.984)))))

